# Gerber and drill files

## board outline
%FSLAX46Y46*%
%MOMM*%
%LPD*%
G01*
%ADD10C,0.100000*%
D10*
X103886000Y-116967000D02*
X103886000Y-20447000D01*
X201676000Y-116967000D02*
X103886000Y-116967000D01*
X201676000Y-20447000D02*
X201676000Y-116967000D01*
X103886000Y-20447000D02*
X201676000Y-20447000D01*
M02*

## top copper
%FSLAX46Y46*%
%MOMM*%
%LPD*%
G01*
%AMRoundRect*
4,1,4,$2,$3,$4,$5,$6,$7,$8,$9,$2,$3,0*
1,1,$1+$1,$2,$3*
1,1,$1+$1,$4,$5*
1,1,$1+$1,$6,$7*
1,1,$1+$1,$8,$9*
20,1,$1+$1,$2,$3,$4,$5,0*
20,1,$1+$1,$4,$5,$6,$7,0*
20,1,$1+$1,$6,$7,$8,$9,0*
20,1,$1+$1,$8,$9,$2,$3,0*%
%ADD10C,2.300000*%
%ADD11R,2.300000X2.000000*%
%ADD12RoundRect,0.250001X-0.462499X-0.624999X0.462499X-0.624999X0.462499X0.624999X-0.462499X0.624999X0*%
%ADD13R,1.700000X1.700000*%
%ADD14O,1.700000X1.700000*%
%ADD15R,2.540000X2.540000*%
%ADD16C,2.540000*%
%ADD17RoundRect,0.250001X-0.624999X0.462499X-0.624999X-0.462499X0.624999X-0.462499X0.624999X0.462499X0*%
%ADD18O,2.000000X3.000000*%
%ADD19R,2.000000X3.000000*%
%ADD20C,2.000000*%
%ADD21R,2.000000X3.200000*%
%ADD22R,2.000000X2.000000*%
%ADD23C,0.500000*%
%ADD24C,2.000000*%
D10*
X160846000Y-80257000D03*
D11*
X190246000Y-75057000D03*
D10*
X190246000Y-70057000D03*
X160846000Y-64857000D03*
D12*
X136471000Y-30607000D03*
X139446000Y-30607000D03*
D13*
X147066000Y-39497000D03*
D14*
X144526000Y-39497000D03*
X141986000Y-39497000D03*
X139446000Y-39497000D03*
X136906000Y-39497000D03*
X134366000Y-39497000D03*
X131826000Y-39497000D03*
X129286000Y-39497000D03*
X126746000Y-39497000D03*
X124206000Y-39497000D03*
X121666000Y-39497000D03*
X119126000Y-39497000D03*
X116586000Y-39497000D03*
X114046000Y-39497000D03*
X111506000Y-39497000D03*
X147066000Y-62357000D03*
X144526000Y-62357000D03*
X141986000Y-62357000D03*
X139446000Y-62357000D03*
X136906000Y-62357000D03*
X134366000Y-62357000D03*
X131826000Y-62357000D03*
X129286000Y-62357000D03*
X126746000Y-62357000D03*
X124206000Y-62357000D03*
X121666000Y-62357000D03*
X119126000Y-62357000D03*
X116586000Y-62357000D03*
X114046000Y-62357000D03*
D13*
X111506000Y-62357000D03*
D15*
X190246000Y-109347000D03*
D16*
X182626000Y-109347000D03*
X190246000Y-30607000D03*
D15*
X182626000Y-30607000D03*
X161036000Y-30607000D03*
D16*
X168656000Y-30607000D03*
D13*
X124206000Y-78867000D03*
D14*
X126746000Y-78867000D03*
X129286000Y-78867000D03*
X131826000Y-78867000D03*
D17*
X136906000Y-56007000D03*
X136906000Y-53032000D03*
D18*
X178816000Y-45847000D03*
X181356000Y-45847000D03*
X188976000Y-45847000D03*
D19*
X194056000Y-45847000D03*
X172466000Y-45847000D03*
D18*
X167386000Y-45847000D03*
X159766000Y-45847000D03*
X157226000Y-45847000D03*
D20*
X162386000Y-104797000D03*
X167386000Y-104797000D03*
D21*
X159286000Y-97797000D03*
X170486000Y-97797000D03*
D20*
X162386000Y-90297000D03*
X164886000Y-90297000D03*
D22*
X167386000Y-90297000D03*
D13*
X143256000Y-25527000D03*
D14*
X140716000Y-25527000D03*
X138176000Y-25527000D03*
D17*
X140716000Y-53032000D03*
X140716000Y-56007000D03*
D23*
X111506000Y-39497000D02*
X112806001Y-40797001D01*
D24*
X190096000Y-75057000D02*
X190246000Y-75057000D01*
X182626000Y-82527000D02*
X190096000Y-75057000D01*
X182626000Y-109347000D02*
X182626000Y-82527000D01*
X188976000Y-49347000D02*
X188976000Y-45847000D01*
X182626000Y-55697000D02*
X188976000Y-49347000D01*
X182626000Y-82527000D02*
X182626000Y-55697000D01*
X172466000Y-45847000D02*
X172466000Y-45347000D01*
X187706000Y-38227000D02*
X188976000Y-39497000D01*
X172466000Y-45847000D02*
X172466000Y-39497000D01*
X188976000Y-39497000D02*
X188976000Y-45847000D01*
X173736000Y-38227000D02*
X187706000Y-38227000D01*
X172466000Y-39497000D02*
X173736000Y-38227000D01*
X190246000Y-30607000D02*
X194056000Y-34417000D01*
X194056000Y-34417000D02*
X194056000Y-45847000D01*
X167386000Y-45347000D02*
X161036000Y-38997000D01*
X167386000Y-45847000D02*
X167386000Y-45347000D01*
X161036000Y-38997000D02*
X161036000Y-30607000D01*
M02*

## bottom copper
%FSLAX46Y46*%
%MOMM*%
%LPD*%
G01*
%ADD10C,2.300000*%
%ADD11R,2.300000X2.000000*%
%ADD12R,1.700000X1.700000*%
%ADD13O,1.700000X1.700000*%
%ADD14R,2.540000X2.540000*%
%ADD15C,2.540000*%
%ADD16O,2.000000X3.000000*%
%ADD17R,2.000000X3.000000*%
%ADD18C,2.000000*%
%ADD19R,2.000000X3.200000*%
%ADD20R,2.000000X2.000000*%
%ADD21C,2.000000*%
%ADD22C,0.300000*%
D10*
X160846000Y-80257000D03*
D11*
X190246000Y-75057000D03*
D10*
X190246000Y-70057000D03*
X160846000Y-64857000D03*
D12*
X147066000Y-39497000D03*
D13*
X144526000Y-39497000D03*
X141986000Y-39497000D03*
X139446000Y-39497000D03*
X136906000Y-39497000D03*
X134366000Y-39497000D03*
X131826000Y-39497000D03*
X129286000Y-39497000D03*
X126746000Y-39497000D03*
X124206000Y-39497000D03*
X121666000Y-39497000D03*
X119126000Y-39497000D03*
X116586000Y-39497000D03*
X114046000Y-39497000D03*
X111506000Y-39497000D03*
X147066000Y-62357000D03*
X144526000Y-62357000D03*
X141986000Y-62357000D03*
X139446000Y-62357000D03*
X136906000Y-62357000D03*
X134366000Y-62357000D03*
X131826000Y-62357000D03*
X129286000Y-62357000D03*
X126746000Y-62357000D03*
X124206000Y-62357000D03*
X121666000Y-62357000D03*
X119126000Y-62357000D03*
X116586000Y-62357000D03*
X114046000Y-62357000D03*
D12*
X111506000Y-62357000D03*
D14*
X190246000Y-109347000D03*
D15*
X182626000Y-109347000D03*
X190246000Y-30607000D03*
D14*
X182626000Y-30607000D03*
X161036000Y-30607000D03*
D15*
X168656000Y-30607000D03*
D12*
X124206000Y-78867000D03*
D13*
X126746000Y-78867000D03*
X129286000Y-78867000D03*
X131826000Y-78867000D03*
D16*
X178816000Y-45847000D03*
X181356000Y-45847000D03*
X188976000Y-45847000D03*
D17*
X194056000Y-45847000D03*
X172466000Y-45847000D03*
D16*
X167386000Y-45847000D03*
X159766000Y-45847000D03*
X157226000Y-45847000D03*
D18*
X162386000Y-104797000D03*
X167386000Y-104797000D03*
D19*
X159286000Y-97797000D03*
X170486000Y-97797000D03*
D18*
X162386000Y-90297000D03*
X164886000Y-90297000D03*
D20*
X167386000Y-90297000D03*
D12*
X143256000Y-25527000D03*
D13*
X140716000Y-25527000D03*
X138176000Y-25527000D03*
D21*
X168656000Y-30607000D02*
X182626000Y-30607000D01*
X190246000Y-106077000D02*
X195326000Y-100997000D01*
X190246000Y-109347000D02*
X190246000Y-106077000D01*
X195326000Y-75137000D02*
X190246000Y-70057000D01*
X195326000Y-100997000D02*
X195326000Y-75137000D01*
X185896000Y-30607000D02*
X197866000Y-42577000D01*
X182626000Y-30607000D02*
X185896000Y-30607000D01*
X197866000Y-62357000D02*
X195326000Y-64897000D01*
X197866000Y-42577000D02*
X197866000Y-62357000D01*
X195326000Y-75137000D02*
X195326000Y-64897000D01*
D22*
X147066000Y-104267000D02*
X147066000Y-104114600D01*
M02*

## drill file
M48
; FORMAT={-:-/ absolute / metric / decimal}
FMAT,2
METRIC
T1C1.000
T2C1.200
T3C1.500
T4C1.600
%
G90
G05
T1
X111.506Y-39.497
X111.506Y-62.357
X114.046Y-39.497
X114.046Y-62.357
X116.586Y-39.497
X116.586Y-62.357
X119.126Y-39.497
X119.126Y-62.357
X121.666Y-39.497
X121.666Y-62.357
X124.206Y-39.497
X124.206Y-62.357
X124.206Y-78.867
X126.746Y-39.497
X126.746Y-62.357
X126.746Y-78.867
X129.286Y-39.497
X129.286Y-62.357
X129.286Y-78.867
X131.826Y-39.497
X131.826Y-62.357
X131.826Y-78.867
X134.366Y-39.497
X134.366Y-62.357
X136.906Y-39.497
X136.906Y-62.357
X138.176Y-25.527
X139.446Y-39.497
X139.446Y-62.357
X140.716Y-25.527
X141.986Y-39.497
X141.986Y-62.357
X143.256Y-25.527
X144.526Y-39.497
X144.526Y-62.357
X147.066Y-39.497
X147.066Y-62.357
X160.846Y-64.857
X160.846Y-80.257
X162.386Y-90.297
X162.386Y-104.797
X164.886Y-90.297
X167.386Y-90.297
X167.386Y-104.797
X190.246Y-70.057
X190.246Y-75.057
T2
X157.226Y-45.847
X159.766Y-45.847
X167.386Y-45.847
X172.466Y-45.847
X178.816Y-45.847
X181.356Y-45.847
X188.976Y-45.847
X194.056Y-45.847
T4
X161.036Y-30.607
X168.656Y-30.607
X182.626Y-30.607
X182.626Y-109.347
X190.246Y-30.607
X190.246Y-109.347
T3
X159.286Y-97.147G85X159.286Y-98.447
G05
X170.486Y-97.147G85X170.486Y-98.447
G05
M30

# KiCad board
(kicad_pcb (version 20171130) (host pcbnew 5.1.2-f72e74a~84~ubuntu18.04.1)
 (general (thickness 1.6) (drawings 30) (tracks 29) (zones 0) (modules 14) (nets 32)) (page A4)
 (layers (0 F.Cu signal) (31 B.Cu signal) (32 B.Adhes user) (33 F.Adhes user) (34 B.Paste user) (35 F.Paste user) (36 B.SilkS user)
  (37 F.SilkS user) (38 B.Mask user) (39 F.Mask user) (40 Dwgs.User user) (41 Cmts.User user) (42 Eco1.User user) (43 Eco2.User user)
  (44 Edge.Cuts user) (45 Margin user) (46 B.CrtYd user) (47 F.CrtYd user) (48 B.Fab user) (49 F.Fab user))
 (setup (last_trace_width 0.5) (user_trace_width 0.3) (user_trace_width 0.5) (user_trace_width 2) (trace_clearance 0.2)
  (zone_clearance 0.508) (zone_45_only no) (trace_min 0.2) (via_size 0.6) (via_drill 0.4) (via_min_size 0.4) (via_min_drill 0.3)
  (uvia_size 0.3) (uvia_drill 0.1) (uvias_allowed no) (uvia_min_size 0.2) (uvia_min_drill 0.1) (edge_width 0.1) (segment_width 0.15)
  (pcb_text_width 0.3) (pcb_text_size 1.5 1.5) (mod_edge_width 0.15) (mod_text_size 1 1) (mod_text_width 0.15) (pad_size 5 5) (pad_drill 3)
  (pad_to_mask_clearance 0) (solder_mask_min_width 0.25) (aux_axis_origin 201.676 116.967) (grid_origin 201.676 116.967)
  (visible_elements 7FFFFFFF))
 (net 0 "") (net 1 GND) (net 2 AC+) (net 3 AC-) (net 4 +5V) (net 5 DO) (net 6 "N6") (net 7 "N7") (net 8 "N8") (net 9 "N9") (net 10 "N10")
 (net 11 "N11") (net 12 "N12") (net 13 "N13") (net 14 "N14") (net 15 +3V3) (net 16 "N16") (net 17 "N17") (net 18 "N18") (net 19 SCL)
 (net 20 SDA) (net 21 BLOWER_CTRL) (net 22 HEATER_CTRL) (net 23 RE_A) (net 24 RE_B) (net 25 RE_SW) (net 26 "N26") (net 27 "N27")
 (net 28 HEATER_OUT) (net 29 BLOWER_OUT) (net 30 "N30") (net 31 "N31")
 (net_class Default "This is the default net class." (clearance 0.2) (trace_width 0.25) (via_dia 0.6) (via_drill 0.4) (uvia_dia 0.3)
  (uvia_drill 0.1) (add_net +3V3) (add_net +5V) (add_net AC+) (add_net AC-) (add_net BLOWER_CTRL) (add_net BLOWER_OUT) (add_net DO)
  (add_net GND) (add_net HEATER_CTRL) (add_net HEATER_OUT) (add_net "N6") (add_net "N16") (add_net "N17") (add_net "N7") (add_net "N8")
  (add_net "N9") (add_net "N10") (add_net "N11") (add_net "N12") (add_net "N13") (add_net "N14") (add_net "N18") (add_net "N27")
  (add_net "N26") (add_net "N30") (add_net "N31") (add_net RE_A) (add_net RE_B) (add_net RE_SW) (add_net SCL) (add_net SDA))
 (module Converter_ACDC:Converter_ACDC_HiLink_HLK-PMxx (layer F.Cu) (at 190.246 75.057 180)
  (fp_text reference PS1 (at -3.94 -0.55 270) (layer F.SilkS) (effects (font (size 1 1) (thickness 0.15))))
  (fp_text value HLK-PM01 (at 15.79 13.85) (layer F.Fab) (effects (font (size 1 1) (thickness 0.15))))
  (pad 3 thru_hole circle (at 29.4 -5.2 180) (size 2.3 2.3) (drill 1) (layers *.Cu *.Mask) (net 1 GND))
  (pad 1 thru_hole rect (at 0 0 180) (size 2.3 2) (drill 1) (layers *.Cu *.Mask) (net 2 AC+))
  (pad 2 thru_hole circle (at 0 5 180) (size 2.3 2.3) (drill 1) (layers *.Cu *.Mask) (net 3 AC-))
  (pad 4 thru_hole circle (at 29.4 10.2 180) (size 2.3 2.3) (drill 1) (layers *.Cu *.Mask) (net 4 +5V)))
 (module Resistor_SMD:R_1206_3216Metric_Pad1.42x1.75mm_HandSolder (layer F.Cu) (at 137.9585 30.607)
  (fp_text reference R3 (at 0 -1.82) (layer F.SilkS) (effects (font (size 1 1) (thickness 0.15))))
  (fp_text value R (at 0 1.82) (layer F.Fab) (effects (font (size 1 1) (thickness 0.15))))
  (pad 1 smd roundrect (at -1.4875 0) (size 1.425 1.75) (layers F.Cu F.Paste F.Mask) (roundrect_rratio 0.175439) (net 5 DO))
  (pad 2 smd roundrect (at 1.4875 0) (size 1.425 1.75) (layers F.Cu F.Paste F.Mask) (roundrect_rratio 0.175439) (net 4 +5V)))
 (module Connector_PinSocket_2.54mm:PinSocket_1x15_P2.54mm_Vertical (layer F.Cu) (at 147.066 39.497 270)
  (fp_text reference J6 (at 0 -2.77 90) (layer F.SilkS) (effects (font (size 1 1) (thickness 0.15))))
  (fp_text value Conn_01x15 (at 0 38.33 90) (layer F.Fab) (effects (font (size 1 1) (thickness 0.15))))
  (pad 1 thru_hole rect (at 0 0 270) (size 1.7 1.7) (drill 1) (layers *.Cu *.Mask) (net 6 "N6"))
  (pad 2 thru_hole oval (at 0 2.54 270) (size 1.7 1.7) (drill 1) (layers *.Cu *.Mask) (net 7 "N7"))
  (pad 3 thru_hole oval (at 0 5.08 270) (size 1.7 1.7) (drill 1) (layers *.Cu *.Mask) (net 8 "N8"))
  (pad 4 thru_hole oval (at 0 7.62 270) (size 1.7 1.7) (drill 1) (layers *.Cu *.Mask) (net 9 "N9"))
  (pad 5 thru_hole oval (at 0 10.16 270) (size 1.7 1.7) (drill 1) (layers *.Cu *.Mask) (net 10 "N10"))
  (pad 6 thru_hole oval (at 0 12.7 270) (size 1.7 1.7) (drill 1) (layers *.Cu *.Mask) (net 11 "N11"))
  (pad 7 thru_hole oval (at 0 15.24 270) (size 1.7 1.7) (drill 1) (layers *.Cu *.Mask) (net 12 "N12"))
  (pad 8 thru_hole oval (at 0 17.78 270) (size 1.7 1.7) (drill 1) (layers *.Cu *.Mask) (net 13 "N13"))
  (pad 9 thru_hole oval (at 0 20.32 270) (size 1.7 1.7) (drill 1) (layers *.Cu *.Mask) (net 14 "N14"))
  (pad 10 thru_hole oval (at 0 22.86 270) (size 1.7 1.7) (drill 1) (layers *.Cu *.Mask) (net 1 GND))
  (pad 11 thru_hole oval (at 0 25.4 270) (size 1.7 1.7) (drill 1) (layers *.Cu *.Mask) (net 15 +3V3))
  (pad 12 thru_hole oval (at 0 27.94 270) (size 1.7 1.7) (drill 1) (layers *.Cu *.Mask) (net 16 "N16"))
  (pad 13 thru_hole oval (at 0 30.48 270) (size 1.7 1.7) (drill 1) (layers *.Cu *.Mask) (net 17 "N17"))
  (pad 14 thru_hole oval (at 0 33.02 270) (size 1.7 1.7) (drill 1) (layers *.Cu *.Mask) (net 1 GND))
  (pad 15 thru_hole oval (at 0 35.56 270) (size 1.7 1.7) (drill 1) (layers *.Cu *.Mask) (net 4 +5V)))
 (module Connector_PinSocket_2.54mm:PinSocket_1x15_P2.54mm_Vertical (layer F.Cu) (at 111.506 62.357 90)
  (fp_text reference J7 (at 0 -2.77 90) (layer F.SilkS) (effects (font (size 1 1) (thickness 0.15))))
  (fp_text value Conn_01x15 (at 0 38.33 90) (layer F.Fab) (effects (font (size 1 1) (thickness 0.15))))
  (pad 15 thru_hole oval (at 0 35.56 90) (size 1.7 1.7) (drill 1) (layers *.Cu *.Mask) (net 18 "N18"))
  (pad 14 thru_hole oval (at 0 33.02 90) (size 1.7 1.7) (drill 1) (layers *.Cu *.Mask) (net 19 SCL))
  (pad 13 thru_hole oval (at 0 30.48 90) (size 1.7 1.7) (drill 1) (layers *.Cu *.Mask) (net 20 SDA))
  (pad 12 thru_hole oval (at 0 27.94 90) (size 1.7 1.7) (drill 1) (layers *.Cu *.Mask) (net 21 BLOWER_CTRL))
  (pad 11 thru_hole oval (at 0 25.4 90) (size 1.7 1.7) (drill 1) (layers *.Cu *.Mask) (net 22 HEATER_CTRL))
  (pad 10 thru_hole oval (at 0 22.86 90) (size 1.7 1.7) (drill 1) (layers *.Cu *.Mask) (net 15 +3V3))
  (pad 9 thru_hole oval (at 0 20.32 90) (size 1.7 1.7) (drill 1) (layers *.Cu *.Mask) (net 1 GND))
  (pad 8 thru_hole oval (at 0 17.78 90) (size 1.7 1.7) (drill 1) (layers *.Cu *.Mask) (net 5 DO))
  (pad 7 thru_hole oval (at 0 15.24 90) (size 1.7 1.7) (drill 1) (layers *.Cu *.Mask) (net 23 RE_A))
  (pad 6 thru_hole oval (at 0 12.7 90) (size 1.7 1.7) (drill 1) (layers *.Cu *.Mask) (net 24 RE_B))
  (pad 5 thru_hole oval (at 0 10.16 90) (size 1.7 1.7) (drill 1) (layers *.Cu *.Mask) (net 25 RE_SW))
  (pad 4 thru_hole oval (at 0 7.62 90) (size 1.7 1.7) (drill 1) (layers *.Cu *.Mask) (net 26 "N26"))
  (pad 3 thru_hole oval (at 0 5.08 90) (size 1.7 1.7) (drill 1) (layers *.Cu *.Mask) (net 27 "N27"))
  (pad 2 thru_hole oval (at 0 2.54 90) (size 1.7 1.7) (drill 1) (layers *.Cu *.Mask) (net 1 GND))
  (pad 1 thru_hole rect (at 0 0 90) (size 1.7 1.7) (drill 1) (layers *.Cu *.Mask) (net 15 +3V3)))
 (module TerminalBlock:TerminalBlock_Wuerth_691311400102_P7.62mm (layer F.Cu) (at 190.246 109.347 180)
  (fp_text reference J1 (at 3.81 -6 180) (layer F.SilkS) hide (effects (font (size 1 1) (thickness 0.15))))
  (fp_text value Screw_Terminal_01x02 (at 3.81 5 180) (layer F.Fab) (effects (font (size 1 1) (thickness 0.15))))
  (pad 1 thru_hole rect (at 0 0 180) (size 2.54 2.54) (drill 1.6) (layers *.Cu *.Mask) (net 3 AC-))
  (pad 2 thru_hole circle (at 7.62 0 180) (size 2.54 2.54) (drill 1.6) (layers *.Cu *.Mask) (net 2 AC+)))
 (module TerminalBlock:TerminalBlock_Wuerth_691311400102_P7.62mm (layer F.Cu) (at 182.626 30.607)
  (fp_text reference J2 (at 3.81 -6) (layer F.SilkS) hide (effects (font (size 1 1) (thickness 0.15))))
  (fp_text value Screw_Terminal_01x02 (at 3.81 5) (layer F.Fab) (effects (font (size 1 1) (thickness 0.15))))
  (pad 2 thru_hole circle (at 7.62 0) (size 2.54 2.54) (drill 1.6) (layers *.Cu *.Mask) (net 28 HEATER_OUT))
  (pad 1 thru_hole rect (at 0 0) (size 2.54 2.54) (drill 1.6) (layers *.Cu *.Mask) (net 3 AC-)))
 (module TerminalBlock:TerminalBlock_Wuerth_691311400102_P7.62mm (layer F.Cu) (at 161.036 30.607)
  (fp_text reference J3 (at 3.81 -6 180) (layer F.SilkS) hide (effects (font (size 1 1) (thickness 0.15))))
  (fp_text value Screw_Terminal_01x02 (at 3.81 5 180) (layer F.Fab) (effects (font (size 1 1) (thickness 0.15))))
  (pad 1 thru_hole rect (at 0 0) (size 2.54 2.54) (drill 1.6) (layers *.Cu *.Mask) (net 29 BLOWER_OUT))
  (pad 2 thru_hole circle (at 7.62 0) (size 2.54 2.54) (drill 1.6) (layers *.Cu *.Mask) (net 3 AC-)))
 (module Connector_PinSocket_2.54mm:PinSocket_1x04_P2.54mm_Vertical (layer F.Cu) (at 124.206 78.867 90)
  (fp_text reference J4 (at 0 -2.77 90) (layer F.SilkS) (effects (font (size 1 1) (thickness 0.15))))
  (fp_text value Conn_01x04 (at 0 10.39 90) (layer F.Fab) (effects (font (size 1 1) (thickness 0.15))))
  (pad 1 thru_hole rect (at 0 0 90) (size 1.7 1.7) (drill 1) (layers *.Cu *.Mask) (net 1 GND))
  (pad 2 thru_hole oval (at 0 2.54 90) (size 1.7 1.7) (drill 1) (layers *.Cu *.Mask) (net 4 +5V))
  (pad 3 thru_hole oval (at 0 5.08 90) (size 1.7 1.7) (drill 1) (layers *.Cu *.Mask) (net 19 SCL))
  (pad 4 thru_hole oval (at 0 7.62 90) (size 1.7 1.7) (drill 1) (layers *.Cu *.Mask) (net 20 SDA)))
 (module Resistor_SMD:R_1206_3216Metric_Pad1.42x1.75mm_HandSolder (layer F.Cu) (at 136.906 54.5195 270)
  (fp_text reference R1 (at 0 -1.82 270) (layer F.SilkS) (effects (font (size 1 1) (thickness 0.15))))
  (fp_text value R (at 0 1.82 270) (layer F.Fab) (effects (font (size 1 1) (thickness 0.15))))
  (pad 2 smd roundrect (at 1.4875 0 270) (size 1.425 1.75) (layers F.Cu F.Paste F.Mask) (roundrect_rratio 0.175439) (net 22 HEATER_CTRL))
  (pad 1 smd roundrect (at -1.4875 0 270) (size 1.425 1.75) (layers F.Cu F.Paste F.Mask) (roundrect_rratio 0.175439) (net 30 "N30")))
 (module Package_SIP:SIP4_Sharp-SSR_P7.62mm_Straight (layer F.Cu) (at 194.056 45.847 180)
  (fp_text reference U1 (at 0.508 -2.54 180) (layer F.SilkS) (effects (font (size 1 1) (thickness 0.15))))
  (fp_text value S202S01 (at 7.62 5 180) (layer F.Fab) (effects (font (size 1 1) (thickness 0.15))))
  (pad 4 thru_hole oval (at 15.24 0 180) (size 2 3) (drill 1.2) (layers *.Cu *.Mask) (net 1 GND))
  (pad 3 thru_hole oval (at 12.7 0 180) (size 2 3) (drill 1.2) (layers *.Cu *.Mask) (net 30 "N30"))
  (pad 2 thru_hole oval (at 5.08 0 180) (size 2 3) (drill 1.2) (layers *.Cu *.Mask) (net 2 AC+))
  (pad 1 thru_hole rect (at 0 0 180) (size 2 3) (drill 1.2) (layers *.Cu *.Mask) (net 28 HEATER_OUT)))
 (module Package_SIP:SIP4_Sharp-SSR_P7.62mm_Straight (layer F.Cu) (at 172.466 45.847 180)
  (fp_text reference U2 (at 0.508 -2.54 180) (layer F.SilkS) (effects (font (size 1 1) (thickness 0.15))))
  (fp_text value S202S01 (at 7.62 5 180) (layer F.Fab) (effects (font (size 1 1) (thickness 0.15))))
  (pad 1 thru_hole rect (at 0 0 180) (size 2 3) (drill 1.2) (layers *.Cu *.Mask) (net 2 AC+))
  (pad 2 thru_hole oval (at 5.08 0 180) (size 2 3) (drill 1.2) (layers *.Cu *.Mask) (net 29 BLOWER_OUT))
  (pad 3 thru_hole oval (at 12.7 0 180) (size 2 3) (drill 1.2) (layers *.Cu *.Mask) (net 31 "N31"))
  (pad 4 thru_hole oval (at 15.24 0 180) (size 2 3) (drill 1.2) (layers *.Cu *.Mask) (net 1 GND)))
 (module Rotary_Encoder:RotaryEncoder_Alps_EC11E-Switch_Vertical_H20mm (layer F.Cu) (at 167.386 90.297 270)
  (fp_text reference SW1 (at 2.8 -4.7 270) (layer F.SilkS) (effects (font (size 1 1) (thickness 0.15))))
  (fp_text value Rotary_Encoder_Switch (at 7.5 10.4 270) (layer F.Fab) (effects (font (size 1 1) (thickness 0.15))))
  (pad S1 thru_hole circle (at 14.5 5 270) (size 2 2) (drill 1) (layers *.Cu *.Mask) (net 25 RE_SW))
  (pad S2 thru_hole circle (at 14.5 0 270) (size 2 2) (drill 1) (layers *.Cu *.Mask) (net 1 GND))
  (pad MP thru_hole rect (at 7.5 8.1 270) (size 3.2 2) (drill oval 2.8 1.5) (layers *.Cu *.Mask))
  (pad MP thru_hole rect (at 7.5 -3.1 270) (size 3.2 2) (drill oval 2.8 1.5) (layers *.Cu *.Mask))
  (pad B thru_hole circle (at 0 5 270) (size 2 2) (drill 1) (layers *.Cu *.Mask) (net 24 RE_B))
  (pad C thru_hole circle (at 0 2.5 270) (size 2 2) (drill 1) (layers *.Cu *.Mask) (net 1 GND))
  (pad A thru_hole rect (at 0 0 270) (size 2 2) (drill 1) (layers *.Cu *.Mask) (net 23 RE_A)))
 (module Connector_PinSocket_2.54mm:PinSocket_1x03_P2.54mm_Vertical (layer F.Cu) (at 143.256 25.527 270)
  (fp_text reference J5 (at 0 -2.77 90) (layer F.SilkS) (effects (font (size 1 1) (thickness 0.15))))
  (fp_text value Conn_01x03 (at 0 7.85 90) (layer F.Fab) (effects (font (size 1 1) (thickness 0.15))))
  (pad 1 thru_hole rect (at 0 0 270) (size 1.7 1.7) (drill 1) (layers *.Cu *.Mask) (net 1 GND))
  (pad 2 thru_hole oval (at 0 2.54 270) (size 1.7 1.7) (drill 1) (layers *.Cu *.Mask) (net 4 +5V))
  (pad 3 thru_hole oval (at 0 5.08 270) (size 1.7 1.7) (drill 1) (layers *.Cu *.Mask) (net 5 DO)))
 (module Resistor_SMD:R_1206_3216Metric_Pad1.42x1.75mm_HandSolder (layer F.Cu) (at 140.716 54.5195 270)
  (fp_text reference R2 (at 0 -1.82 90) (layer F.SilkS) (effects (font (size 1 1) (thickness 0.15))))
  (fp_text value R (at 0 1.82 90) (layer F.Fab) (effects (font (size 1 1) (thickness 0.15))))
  (pad 1 smd roundrect (at -1.4875 0 270) (size 1.425 1.75) (layers F.Cu F.Paste F.Mask) (roundrect_rratio 0.175439) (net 31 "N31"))
  (pad 2 smd roundrect (at 1.4875 0 270) (size 1.425 1.75) (layers F.Cu F.Paste F.Mask) (roundrect_rratio 0.175439) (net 21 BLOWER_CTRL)))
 (gr_line (start 103.886 116.967) (end 103.886 20.447) (layer Edge.Cuts) (width 0.1))
 (gr_line (start 201.676 116.967) (end 103.886 116.967) (layer Edge.Cuts) (width 0.1))
 (gr_line (start 201.676 20.447) (end 201.676 116.967) (layer Edge.Cuts) (width 0.1))
 (gr_line (start 103.886 20.447) (end 201.676 20.447) (layer Edge.Cuts) (width 0.1))
 (segment (start 111.506 39.497) (end 112.806001 40.797001) (width 0.5) (layer F.Cu) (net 4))
 (segment (start 168.656 30.607) (end 182.626 30.607) (width 2) (layer B.Cu) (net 3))
 (segment (start 190.246 106.077) (end 195.326 100.997) (width 2) (layer B.Cu) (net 3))
 (segment (start 190.246 109.347) (end 190.246 106.077) (width 2) (layer B.Cu) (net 3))
 (segment (start 195.326 75.137) (end 190.246 70.057) (width 2) (layer B.Cu) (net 3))
 (segment (start 195.326 100.997) (end 195.326 75.137) (width 2) (layer B.Cu) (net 3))
 (segment (start 185.896 30.607) (end 197.866 42.577) (width 2) (layer B.Cu) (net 3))
 (segment (start 182.626 30.607) (end 185.896 30.607) (width 2) (layer B.Cu) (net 3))
 (segment (start 197.866 62.357) (end 195.326 64.897) (width 2) (layer B.Cu) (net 3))
 (segment (start 197.866 42.577) (end 197.866 62.357) (width 2) (layer B.Cu) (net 3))
 (segment (start 195.326 75.137) (end 195.326 64.897) (width 2) (layer B.Cu) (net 3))
 (segment (start 190.096 75.057) (end 190.246 75.057) (width 2) (layer F.Cu) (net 2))
 (segment (start 182.626 82.527) (end 190.096 75.057) (width 2) (layer F.Cu) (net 2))
 (segment (start 182.626 109.347) (end 182.626 82.527) (width 2) (layer F.Cu) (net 2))
 (segment (start 188.976 49.347) (end 188.976 45.847) (width 2) (layer F.Cu) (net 2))
 (segment (start 182.626 55.697) (end 188.976 49.347) (width 2) (layer F.Cu) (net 2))
 (segment (start 182.626 82.527) (end 182.626 55.697) (width 2) (layer F.Cu) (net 2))
 (segment (start 172.466 45.847) (end 172.466 45.347) (width 2) (layer F.Cu) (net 2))
 (segment (start 187.706 38.227) (end 188.976 39.497) (width 2) (layer F.Cu) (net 2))
 (segment (start 172.466 45.847) (end 172.466 39.497) (width 2) (layer F.Cu) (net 2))
 (segment (start 188.976 39.497) (end 188.976 45.847) (width 2) (layer F.Cu) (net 2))
 (segment (start 173.736 38.227) (end 187.706 38.227) (width 2) (layer F.Cu) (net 2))
 (segment (start 172.466 39.497) (end 173.736 38.227) (width 2) (layer F.Cu) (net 2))
 (segment (start 190.246 30.607) (end 194.056 34.417) (width 2) (layer F.Cu) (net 28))
 (segment (start 194.056 34.417) (end 194.056 45.847) (width 2) (layer F.Cu) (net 28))
 (segment (start 167.386 45.347) (end 161.036 38.997) (width 2) (layer F.Cu) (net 29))
 (segment (start 167.386 45.847) (end 167.386 45.347) (width 2) (layer F.Cu) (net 29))
 (segment (start 161.036 38.997) (end 161.036 30.607) (width 2) (layer F.Cu) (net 29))
 (segment (start 147.066 104.267) (end 147.066 104.1146) (width 0.3) (layer B.Cu) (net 24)))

